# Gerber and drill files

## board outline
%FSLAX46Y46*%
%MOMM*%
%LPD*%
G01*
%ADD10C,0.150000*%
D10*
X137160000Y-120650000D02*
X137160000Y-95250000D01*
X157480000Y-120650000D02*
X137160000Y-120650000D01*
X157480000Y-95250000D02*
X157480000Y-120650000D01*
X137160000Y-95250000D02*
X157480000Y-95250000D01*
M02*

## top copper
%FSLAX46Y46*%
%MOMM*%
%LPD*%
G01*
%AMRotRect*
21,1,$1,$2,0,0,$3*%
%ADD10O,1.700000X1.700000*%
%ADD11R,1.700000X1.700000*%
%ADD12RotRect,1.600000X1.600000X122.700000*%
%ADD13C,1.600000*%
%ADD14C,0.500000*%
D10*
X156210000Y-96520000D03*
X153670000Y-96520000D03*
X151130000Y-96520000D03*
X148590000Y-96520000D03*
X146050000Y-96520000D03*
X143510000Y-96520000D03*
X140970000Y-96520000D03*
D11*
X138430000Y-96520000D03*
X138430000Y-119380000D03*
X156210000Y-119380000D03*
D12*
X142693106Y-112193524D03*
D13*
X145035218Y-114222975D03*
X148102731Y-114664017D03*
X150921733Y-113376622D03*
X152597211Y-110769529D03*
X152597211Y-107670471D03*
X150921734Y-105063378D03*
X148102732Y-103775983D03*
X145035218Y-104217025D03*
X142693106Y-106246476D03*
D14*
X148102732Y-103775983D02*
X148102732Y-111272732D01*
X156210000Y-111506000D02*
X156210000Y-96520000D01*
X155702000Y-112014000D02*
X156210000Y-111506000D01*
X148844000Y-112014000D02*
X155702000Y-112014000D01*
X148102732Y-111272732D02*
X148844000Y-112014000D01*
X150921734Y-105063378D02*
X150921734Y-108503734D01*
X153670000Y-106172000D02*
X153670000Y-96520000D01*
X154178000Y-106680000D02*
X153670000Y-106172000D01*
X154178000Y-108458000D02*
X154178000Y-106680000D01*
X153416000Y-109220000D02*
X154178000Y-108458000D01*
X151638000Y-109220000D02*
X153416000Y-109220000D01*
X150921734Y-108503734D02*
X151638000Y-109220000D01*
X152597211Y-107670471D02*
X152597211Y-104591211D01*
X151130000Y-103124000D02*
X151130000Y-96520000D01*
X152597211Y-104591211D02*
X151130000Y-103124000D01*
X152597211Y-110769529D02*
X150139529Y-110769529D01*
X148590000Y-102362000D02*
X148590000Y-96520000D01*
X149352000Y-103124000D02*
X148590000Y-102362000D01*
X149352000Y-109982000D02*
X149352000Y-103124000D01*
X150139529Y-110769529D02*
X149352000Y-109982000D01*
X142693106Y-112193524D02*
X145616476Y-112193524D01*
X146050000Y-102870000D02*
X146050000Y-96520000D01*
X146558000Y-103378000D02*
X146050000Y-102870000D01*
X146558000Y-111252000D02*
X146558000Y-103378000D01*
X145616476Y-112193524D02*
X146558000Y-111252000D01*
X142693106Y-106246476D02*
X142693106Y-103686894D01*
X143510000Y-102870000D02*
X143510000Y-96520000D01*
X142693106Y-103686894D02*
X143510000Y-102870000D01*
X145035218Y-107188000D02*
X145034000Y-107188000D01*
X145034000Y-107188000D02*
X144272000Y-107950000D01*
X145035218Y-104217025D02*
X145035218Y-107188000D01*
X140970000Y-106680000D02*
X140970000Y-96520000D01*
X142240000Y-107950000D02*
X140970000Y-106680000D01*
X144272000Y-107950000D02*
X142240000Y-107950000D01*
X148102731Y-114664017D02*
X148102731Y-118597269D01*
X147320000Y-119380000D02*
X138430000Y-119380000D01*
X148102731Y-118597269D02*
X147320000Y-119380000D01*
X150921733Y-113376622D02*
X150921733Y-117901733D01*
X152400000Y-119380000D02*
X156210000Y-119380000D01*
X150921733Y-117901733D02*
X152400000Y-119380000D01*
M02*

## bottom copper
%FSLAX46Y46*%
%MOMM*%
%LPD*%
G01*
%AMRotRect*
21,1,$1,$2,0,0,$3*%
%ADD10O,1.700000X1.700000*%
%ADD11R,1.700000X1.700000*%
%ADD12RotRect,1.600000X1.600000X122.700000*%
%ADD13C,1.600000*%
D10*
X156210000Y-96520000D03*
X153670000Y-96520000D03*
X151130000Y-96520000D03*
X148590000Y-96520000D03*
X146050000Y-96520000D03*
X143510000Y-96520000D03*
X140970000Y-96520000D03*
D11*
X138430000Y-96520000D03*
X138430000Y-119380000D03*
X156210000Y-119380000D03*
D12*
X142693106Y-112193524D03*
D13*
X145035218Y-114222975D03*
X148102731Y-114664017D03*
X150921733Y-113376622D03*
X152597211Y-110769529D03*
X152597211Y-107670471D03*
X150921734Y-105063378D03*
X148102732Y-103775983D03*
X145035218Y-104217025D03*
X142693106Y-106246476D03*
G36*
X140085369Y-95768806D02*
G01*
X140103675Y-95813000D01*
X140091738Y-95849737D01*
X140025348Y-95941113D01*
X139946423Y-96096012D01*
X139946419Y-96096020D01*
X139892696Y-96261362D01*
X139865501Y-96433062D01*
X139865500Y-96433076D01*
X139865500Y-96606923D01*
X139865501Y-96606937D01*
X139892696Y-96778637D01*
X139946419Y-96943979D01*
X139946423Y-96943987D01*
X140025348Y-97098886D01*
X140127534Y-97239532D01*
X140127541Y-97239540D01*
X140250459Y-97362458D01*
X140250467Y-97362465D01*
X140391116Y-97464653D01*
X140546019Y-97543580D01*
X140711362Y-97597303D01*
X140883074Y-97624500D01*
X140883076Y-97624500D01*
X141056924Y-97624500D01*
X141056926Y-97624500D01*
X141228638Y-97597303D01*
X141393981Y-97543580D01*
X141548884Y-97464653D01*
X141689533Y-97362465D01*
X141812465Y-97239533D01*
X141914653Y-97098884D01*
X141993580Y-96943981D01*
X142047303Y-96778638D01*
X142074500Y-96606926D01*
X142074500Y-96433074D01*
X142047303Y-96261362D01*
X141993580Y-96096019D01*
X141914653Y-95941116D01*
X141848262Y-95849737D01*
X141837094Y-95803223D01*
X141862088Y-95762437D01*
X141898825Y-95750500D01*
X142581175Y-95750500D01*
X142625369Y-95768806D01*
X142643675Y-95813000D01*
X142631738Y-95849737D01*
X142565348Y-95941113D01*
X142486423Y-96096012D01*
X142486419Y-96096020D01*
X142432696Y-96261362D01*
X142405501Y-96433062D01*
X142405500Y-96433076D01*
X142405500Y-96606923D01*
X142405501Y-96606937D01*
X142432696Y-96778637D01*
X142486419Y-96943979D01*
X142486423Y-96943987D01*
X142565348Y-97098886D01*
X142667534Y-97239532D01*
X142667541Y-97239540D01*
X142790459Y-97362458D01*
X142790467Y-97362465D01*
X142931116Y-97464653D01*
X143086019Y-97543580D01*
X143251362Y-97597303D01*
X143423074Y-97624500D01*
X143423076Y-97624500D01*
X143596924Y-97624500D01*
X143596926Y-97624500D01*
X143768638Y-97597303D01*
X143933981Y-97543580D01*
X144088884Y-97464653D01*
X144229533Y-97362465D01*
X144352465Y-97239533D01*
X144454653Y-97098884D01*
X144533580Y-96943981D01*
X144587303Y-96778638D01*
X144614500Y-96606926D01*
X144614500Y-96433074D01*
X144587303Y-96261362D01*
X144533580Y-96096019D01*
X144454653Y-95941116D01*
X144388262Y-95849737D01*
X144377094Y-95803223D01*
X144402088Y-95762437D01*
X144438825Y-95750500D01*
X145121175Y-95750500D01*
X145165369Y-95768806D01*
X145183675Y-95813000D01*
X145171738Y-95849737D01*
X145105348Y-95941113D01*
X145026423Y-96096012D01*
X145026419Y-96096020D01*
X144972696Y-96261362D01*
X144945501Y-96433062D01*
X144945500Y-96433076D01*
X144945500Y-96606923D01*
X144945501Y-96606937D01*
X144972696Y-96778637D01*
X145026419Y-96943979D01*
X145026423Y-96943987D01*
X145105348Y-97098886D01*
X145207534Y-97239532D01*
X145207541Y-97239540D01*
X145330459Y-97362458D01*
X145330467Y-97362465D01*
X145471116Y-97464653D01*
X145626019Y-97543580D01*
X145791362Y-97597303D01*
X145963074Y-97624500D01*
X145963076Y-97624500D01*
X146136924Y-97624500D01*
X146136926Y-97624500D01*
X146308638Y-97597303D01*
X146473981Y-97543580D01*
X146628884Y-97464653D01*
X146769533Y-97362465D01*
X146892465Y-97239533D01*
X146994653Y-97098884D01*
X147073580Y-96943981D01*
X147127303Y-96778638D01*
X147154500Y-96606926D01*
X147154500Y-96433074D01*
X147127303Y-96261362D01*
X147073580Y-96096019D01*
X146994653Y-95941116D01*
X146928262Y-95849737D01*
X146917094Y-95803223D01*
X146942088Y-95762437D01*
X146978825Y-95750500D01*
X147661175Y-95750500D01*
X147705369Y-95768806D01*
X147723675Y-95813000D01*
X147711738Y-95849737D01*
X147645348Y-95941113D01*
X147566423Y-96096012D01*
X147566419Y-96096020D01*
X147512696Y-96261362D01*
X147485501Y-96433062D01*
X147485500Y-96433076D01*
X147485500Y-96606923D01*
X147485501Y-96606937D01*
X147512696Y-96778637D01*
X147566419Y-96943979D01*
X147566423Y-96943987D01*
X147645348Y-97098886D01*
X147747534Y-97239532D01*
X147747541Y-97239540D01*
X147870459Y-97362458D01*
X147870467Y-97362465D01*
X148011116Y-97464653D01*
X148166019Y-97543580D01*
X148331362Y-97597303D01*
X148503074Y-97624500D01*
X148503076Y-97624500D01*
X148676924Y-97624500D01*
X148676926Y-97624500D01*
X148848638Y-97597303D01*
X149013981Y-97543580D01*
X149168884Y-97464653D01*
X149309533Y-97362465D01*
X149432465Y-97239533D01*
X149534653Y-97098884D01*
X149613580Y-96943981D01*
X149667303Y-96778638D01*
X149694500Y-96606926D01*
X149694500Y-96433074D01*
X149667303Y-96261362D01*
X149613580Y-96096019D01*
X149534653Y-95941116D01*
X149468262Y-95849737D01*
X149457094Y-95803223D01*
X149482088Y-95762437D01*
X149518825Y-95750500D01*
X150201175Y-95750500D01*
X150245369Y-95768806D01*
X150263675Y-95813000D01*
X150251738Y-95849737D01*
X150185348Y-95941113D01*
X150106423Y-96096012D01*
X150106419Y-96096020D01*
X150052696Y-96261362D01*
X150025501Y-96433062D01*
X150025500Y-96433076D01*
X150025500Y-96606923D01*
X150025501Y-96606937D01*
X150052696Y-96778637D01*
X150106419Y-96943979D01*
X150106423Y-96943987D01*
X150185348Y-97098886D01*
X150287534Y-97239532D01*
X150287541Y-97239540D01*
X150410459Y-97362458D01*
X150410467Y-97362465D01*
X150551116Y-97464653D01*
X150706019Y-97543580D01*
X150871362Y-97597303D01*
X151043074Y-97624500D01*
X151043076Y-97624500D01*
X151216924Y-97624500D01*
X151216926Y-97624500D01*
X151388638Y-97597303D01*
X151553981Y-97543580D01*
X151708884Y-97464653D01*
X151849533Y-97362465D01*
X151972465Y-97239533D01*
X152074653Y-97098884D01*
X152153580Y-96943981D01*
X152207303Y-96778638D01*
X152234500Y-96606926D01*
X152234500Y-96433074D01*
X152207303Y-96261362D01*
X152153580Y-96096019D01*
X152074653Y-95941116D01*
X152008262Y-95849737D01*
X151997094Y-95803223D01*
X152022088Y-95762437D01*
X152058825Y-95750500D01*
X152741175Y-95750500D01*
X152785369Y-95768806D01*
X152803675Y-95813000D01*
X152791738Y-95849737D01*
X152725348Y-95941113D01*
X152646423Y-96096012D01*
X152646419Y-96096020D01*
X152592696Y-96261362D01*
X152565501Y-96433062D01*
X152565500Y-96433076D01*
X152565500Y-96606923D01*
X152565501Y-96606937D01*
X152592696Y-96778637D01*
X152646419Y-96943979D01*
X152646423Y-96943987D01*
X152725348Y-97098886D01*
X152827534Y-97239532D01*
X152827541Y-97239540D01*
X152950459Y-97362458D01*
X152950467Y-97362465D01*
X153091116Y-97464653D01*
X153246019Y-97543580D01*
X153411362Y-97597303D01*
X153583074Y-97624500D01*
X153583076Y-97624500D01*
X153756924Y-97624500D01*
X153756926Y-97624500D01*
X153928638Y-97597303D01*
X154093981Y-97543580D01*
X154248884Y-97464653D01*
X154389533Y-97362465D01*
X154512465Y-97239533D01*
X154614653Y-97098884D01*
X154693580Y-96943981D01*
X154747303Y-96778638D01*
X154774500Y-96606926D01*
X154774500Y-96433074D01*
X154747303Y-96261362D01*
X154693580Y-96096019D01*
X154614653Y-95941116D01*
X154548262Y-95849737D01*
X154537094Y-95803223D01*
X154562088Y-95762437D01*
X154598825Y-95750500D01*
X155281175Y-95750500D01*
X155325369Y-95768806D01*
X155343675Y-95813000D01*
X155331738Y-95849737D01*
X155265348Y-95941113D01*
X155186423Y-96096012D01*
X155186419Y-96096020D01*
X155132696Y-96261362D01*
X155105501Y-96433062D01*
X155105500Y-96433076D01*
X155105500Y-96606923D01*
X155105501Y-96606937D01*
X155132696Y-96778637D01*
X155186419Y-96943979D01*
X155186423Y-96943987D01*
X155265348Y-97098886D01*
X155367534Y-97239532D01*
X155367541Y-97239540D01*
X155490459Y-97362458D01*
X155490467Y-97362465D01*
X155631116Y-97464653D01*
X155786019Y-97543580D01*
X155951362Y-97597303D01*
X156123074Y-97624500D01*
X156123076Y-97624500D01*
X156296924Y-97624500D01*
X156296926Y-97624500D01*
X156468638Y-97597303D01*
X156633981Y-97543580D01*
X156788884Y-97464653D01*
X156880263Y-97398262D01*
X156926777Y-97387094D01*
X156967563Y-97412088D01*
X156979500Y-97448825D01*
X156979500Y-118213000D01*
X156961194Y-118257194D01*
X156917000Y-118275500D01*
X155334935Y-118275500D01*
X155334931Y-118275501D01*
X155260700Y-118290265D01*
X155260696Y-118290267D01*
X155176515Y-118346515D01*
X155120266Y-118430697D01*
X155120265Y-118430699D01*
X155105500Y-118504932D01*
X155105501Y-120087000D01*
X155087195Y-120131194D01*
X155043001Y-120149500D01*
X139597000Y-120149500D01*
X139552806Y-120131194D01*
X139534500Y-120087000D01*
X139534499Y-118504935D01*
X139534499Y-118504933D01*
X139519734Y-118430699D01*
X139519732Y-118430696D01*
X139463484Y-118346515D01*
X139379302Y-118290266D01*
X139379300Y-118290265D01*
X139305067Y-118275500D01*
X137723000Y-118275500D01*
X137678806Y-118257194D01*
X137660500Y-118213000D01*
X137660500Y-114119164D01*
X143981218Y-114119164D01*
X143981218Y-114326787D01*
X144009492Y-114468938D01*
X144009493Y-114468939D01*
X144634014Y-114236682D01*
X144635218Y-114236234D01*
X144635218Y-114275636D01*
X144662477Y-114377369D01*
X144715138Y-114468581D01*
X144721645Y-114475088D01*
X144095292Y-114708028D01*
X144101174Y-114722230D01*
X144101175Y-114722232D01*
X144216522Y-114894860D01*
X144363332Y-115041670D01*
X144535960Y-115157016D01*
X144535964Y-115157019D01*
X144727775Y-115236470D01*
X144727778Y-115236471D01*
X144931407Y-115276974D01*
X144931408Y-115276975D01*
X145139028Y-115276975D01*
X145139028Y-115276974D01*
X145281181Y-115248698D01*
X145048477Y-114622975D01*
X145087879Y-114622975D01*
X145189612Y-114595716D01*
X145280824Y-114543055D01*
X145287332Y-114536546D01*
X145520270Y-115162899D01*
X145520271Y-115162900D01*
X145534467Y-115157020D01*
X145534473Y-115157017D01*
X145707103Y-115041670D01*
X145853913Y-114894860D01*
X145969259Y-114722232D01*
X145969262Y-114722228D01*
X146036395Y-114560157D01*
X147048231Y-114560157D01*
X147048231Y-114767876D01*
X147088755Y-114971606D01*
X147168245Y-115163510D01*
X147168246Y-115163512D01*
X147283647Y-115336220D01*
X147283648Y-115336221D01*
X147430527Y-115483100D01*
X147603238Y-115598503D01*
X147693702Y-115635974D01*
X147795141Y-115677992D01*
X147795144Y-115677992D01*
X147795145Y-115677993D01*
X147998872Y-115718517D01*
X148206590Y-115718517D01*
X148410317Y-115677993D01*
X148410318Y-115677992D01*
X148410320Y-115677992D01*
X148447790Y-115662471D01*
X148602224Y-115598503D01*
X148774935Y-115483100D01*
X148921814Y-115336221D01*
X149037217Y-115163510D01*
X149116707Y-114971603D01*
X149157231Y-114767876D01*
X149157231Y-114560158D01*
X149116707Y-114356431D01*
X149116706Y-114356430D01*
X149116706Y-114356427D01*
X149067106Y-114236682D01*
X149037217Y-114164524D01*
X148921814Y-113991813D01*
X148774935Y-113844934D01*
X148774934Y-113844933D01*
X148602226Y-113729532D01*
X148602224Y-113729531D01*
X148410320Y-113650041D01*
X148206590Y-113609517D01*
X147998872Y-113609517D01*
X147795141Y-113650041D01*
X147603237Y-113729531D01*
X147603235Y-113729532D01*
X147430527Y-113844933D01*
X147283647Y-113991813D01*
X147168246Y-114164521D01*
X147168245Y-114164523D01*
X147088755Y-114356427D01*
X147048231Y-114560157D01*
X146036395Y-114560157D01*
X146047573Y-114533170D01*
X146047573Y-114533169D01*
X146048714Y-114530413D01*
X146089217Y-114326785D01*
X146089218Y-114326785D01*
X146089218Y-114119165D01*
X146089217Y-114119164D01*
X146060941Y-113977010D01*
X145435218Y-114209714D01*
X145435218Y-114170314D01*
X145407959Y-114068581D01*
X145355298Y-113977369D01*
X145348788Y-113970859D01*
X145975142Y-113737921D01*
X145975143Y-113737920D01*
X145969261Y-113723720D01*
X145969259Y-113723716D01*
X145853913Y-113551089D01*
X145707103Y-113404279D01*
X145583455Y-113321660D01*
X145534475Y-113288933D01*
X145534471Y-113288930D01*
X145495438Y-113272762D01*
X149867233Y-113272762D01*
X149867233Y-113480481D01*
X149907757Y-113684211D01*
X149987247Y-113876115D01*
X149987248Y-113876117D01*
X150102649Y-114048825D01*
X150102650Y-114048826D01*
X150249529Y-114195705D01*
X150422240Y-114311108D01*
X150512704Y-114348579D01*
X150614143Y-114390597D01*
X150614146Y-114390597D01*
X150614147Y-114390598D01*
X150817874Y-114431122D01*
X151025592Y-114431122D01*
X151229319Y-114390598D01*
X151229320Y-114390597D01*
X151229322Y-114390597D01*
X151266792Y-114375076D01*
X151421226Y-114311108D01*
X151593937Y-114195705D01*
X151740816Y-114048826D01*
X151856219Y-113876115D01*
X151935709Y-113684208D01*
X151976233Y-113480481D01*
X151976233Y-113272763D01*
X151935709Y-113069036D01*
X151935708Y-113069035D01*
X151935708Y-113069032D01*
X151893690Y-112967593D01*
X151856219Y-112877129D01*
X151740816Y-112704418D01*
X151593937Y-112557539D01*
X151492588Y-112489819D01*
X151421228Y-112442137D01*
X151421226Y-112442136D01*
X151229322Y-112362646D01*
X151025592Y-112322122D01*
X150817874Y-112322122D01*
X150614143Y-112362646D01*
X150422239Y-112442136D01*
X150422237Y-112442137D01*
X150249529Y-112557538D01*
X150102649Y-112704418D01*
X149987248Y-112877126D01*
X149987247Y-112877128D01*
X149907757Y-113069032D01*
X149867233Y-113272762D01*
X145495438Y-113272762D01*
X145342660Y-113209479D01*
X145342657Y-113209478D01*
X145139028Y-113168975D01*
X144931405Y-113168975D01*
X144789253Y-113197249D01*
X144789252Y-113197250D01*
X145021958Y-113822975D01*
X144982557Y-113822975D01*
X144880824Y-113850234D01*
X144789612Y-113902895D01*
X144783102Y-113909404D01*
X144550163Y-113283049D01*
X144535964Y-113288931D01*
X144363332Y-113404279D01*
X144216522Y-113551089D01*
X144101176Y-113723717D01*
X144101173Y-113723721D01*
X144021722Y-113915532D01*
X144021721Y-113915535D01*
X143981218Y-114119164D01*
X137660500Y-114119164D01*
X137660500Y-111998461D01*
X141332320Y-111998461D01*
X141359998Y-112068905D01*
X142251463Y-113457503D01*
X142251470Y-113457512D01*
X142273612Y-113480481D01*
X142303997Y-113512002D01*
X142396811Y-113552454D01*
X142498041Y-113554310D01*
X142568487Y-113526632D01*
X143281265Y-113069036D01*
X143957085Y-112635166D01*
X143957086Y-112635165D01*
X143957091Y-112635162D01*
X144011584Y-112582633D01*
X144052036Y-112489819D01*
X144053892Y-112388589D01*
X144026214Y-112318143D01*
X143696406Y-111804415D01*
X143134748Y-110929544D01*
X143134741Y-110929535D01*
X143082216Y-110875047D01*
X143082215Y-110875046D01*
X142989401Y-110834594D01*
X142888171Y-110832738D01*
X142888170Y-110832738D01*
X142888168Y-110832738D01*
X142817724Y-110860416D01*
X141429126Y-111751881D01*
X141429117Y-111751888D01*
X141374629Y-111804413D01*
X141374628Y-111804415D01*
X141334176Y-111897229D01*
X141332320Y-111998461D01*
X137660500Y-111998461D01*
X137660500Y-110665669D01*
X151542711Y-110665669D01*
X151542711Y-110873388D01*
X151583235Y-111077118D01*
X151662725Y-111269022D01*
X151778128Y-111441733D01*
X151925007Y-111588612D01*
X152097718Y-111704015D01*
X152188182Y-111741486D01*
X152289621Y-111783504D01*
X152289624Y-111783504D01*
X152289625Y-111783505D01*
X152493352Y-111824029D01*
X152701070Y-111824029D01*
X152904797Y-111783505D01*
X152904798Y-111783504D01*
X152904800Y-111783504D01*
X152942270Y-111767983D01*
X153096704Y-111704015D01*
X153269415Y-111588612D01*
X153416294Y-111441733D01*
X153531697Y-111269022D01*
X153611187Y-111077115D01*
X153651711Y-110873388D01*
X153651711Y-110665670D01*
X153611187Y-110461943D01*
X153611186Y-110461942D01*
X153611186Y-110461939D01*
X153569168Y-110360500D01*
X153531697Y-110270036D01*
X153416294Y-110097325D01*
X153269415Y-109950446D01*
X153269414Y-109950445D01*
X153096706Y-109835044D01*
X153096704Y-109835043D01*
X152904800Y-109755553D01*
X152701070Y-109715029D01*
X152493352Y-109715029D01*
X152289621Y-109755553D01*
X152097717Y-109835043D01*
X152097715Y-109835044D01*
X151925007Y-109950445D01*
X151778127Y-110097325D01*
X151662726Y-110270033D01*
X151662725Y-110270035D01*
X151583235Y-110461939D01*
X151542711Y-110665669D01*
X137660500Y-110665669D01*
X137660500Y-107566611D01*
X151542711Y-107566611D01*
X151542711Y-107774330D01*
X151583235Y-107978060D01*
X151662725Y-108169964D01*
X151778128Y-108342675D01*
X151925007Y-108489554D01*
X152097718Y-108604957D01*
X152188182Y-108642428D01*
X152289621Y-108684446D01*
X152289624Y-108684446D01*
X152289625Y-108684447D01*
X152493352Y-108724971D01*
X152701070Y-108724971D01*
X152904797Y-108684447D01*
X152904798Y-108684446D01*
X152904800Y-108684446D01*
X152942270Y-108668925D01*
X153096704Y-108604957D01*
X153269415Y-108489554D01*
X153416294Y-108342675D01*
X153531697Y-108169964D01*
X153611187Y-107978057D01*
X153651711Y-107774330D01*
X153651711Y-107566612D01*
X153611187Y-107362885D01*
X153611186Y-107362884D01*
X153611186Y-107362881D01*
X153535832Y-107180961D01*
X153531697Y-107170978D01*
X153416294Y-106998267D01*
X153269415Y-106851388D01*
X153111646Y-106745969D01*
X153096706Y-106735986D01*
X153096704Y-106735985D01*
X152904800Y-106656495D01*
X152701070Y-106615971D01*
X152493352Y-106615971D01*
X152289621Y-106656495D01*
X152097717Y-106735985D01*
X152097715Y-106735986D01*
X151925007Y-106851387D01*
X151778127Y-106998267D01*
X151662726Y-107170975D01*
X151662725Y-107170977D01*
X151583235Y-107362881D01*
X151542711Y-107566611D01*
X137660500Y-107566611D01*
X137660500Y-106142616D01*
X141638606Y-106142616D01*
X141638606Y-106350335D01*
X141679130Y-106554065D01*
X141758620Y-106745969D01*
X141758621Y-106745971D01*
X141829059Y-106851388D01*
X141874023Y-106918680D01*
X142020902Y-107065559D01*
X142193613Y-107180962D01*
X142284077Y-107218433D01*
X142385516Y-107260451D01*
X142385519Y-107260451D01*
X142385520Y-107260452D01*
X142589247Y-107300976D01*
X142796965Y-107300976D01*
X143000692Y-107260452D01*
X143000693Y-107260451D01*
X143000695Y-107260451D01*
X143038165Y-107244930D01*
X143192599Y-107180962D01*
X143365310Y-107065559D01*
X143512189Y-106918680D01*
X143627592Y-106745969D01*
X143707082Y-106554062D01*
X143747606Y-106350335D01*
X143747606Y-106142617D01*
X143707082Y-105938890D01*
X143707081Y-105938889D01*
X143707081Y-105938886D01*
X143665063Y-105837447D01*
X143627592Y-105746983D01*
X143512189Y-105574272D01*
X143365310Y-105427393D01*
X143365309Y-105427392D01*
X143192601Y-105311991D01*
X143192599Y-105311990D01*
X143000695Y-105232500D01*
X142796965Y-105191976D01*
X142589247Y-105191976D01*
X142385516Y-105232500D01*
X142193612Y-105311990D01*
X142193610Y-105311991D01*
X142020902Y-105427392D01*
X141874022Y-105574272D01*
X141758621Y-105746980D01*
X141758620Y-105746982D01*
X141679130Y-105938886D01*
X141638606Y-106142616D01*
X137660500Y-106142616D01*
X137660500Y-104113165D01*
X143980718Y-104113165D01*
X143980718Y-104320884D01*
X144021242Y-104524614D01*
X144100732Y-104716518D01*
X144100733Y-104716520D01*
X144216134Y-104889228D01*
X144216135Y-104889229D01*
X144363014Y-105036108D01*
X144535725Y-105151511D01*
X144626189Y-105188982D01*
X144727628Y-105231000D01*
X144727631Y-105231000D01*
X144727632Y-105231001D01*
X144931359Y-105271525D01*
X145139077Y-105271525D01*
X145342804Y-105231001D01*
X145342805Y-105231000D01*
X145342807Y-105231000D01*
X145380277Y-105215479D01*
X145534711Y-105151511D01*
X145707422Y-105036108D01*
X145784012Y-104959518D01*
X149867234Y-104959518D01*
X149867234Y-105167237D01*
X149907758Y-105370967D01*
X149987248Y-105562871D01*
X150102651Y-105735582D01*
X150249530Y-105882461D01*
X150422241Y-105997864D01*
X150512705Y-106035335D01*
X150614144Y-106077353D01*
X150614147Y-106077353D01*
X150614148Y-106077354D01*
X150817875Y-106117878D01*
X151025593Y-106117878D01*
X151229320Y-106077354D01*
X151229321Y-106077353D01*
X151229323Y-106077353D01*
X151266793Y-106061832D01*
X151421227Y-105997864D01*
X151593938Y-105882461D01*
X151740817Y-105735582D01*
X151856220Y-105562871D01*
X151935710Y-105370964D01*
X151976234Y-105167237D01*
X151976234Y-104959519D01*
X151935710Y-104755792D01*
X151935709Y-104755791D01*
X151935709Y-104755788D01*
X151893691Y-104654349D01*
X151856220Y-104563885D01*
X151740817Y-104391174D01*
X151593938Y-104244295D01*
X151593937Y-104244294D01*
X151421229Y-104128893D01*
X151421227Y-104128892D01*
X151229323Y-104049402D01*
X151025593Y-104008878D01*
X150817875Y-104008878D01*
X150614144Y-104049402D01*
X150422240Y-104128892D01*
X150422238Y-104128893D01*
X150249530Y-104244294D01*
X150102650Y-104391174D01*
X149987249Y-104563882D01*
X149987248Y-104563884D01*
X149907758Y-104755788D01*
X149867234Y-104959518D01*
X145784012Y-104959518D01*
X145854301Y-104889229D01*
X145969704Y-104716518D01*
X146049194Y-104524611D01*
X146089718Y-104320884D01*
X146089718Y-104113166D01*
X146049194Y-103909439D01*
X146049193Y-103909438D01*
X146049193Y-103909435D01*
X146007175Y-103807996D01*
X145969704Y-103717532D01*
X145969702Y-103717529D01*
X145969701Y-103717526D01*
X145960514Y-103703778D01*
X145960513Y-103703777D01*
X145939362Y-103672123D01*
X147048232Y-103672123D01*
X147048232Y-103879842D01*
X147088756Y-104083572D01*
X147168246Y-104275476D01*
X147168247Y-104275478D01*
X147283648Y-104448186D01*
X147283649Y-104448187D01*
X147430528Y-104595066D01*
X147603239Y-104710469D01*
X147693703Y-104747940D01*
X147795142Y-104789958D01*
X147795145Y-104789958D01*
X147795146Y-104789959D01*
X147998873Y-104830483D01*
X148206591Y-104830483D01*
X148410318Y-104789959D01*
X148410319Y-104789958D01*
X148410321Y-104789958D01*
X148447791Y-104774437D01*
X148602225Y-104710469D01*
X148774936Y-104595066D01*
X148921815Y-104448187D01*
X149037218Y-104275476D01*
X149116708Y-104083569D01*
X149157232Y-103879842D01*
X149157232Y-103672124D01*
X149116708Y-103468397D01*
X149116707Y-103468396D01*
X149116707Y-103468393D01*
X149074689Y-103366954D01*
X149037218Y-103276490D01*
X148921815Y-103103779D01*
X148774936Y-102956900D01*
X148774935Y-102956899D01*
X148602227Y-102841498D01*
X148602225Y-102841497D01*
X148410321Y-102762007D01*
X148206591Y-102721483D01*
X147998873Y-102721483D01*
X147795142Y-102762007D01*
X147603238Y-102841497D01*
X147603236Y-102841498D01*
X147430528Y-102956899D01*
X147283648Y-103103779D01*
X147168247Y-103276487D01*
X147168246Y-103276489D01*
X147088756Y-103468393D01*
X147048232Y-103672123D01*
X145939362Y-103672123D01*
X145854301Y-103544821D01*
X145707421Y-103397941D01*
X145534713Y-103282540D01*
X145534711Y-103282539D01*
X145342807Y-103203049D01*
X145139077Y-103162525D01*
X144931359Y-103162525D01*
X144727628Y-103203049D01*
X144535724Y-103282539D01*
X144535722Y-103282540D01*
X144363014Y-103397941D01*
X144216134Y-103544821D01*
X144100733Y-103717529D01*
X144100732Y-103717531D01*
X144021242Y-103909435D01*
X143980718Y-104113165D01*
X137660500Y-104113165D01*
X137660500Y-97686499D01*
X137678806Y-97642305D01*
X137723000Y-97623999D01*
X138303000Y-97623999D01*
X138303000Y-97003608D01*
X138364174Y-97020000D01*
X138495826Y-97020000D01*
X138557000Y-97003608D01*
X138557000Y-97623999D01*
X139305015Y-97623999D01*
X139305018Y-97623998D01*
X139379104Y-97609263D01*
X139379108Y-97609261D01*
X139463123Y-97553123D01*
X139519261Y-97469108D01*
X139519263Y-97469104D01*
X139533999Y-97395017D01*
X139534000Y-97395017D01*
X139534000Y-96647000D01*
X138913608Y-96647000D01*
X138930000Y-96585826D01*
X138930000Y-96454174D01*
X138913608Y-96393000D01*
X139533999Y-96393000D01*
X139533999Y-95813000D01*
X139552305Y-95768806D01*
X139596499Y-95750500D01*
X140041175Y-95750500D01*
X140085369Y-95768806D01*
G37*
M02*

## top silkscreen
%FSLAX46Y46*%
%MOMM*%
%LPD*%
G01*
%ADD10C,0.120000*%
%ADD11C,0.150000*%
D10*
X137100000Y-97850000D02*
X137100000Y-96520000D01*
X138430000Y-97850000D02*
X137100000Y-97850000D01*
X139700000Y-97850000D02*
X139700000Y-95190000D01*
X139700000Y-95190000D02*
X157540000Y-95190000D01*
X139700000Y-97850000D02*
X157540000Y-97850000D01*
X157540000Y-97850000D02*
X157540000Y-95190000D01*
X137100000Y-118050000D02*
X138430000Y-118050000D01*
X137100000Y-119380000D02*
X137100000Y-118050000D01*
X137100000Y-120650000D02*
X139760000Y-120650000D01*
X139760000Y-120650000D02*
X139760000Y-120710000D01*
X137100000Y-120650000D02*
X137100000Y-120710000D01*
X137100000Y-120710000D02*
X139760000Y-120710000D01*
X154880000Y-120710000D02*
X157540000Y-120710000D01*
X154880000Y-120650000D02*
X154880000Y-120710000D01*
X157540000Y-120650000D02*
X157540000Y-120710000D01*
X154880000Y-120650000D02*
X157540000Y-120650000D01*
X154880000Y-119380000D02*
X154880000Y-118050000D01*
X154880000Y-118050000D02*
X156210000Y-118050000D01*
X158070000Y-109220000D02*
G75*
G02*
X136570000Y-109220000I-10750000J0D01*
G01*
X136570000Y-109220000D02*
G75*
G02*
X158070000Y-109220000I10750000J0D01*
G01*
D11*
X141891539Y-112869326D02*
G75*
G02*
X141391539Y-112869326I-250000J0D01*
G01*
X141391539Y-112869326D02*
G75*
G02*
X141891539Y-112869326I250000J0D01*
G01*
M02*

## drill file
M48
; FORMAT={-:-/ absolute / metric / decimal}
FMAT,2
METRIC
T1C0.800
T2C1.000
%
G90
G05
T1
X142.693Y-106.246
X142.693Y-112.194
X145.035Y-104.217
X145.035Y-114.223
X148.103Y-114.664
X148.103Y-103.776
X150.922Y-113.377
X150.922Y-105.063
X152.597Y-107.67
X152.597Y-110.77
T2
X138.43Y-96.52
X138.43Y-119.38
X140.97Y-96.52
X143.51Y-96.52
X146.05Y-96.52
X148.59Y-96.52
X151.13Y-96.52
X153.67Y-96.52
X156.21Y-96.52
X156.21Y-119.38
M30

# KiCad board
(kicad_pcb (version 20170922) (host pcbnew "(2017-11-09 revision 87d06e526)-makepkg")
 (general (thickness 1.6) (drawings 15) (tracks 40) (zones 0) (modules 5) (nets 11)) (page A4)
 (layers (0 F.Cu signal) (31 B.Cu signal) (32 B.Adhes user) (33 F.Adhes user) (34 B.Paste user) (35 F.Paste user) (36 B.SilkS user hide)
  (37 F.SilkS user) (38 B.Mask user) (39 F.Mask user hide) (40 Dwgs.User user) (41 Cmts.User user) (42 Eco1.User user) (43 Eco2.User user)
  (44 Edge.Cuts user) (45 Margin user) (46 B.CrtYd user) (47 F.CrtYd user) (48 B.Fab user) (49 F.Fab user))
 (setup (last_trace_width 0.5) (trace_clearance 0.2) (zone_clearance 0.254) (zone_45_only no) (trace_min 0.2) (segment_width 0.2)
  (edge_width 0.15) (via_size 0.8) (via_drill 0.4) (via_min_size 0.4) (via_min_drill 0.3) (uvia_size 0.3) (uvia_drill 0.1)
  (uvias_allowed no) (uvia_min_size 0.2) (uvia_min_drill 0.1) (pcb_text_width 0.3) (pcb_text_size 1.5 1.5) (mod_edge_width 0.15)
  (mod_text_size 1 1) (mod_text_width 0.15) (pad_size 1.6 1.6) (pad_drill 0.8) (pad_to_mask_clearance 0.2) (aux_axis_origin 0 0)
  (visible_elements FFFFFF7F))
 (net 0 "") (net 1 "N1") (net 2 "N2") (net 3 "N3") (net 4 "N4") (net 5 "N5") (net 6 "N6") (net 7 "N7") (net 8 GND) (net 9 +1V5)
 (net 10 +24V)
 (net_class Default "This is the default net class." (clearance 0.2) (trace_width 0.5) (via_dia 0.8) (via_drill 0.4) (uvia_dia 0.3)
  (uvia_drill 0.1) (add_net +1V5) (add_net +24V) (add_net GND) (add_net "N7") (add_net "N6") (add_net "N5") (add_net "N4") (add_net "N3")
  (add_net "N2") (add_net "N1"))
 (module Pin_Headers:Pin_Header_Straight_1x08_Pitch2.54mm (layer F.Cu) (at 138.43 96.52 90)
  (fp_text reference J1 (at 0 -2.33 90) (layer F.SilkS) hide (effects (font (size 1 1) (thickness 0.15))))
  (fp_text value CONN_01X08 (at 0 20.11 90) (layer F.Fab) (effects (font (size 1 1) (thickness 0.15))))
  (fp_line (start -1.33 -1.33) (end 0 -1.33) (layer F.SilkS) (width 0.12))
  (fp_line (start -1.33 0) (end -1.33 -1.33) (layer F.SilkS) (width 0.12))
  (fp_line (start -1.33 1.27) (end 1.33 1.27) (layer F.SilkS) (width 0.12))
  (fp_line (start 1.33 1.27) (end 1.33 19.11) (layer F.SilkS) (width 0.12))
  (fp_line (start -1.33 1.27) (end -1.33 19.11) (layer F.SilkS) (width 0.12))
  (fp_line (start -1.33 19.11) (end 1.33 19.11) (layer F.SilkS) (width 0.12))
  (pad 8 thru_hole oval (at 0 17.78 90) (size 1.7 1.7) (drill 1) (layers *.Cu *.Mask) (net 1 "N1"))
  (pad 7 thru_hole oval (at 0 15.24 90) (size 1.7 1.7) (drill 1) (layers *.Cu *.Mask) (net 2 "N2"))
  (pad 6 thru_hole oval (at 0 12.7 90) (size 1.7 1.7) (drill 1) (layers *.Cu *.Mask) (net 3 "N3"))
  (pad 5 thru_hole oval (at 0 10.16 90) (size 1.7 1.7) (drill 1) (layers *.Cu *.Mask) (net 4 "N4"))
  (pad 4 thru_hole oval (at 0 7.62 90) (size 1.7 1.7) (drill 1) (layers *.Cu *.Mask) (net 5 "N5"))
  (pad 3 thru_hole oval (at 0 5.08 90) (size 1.7 1.7) (drill 1) (layers *.Cu *.Mask) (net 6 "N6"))
  (pad 2 thru_hole oval (at 0 2.54 90) (size 1.7 1.7) (drill 1) (layers *.Cu *.Mask) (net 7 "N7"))
  (pad 1 thru_hole rect (at 0 0 90) (size 1.7 1.7) (drill 1) (layers *.Cu *.Mask) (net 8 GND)))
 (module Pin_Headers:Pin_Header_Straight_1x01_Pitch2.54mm (layer F.Cu) (at 138.43 119.38)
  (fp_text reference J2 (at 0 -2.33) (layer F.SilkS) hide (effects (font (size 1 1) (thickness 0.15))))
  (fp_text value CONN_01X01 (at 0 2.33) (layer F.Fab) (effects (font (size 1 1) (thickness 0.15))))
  (fp_line (start -1.33 -1.33) (end 0 -1.33) (layer F.SilkS) (width 0.12))
  (fp_line (start -1.33 0) (end -1.33 -1.33) (layer F.SilkS) (width 0.12))
  (fp_line (start -1.33 1.27) (end 1.33 1.27) (layer F.SilkS) (width 0.12))
  (fp_line (start 1.33 1.27) (end 1.33 1.33) (layer F.SilkS) (width 0.12))
  (fp_line (start -1.33 1.27) (end -1.33 1.33) (layer F.SilkS) (width 0.12))
  (fp_line (start -1.33 1.33) (end 1.33 1.33) (layer F.SilkS) (width 0.12))
  (pad 1 thru_hole rect (at 0 0) (size 1.7 1.7) (drill 1) (layers *.Cu *.Mask) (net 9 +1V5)))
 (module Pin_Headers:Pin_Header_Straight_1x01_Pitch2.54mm (layer F.Cu) (at 156.21 119.38)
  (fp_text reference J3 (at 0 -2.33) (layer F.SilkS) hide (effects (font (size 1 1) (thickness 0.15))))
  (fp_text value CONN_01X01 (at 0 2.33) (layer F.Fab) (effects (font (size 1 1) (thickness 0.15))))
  (fp_line (start -1.33 1.33) (end 1.33 1.33) (layer F.SilkS) (width 0.12))
  (fp_line (start -1.33 1.27) (end -1.33 1.33) (layer F.SilkS) (width 0.12))
  (fp_line (start 1.33 1.27) (end 1.33 1.33) (layer F.SilkS) (width 0.12))
  (fp_line (start -1.33 1.27) (end 1.33 1.27) (layer F.SilkS) (width 0.12))
  (fp_line (start -1.33 0) (end -1.33 -1.33) (layer F.SilkS) (width 0.12))
  (fp_line (start -1.33 -1.33) (end 0 -1.33) (layer F.SilkS) (width 0.12))
  (pad 1 thru_hole rect (at 0 0) (size 1.7 1.7) (drill 1) (layers *.Cu *.Mask) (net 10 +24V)))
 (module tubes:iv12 (layer F.Cu) (at 147.32 109.22 90)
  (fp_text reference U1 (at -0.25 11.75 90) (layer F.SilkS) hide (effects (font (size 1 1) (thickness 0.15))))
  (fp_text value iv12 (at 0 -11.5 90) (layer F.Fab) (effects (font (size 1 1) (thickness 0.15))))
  (fp_circle (center 0 0) (end 10.75 0) (layer F.SilkS) (width 0.12))
  (fp_circle (center -3.649326 -5.678461) (end -3.514165 -5.468148) (layer F.SilkS) (width 0.15))
  (pad 1 thru_hole rect (at -2.973524 -4.626894 122.7) (size 1.6 1.6) (drill 0.8) (layers *.Cu *.Mask) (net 5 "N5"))
  (pad 2 thru_hole circle (at -5.002975 -2.284782 155.4) (size 1.6 1.6) (drill 0.8) (layers *.Cu *.Mask) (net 8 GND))
  (pad 3 thru_hole circle (at -5.444017 0.782731 188.2) (size 1.6 1.6) (drill 0.8) (layers *.Cu *.Mask) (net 9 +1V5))
  (pad 4 thru_hole circle (at -4.156622 3.601733 220.9) (size 1.6 1.6) (drill 0.8) (layers *.Cu *.Mask) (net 10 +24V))
  (pad 5 thru_hole circle (at -1.549529 5.277211 253.6) (size 1.6 1.6) (drill 0.8) (layers *.Cu *.Mask) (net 4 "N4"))
  (pad 6 thru_hole circle (at 1.549529 5.277211 286.3) (size 1.6 1.6) (drill 0.8) (layers *.Cu *.Mask) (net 3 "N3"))
  (pad 7 thru_hole circle (at 4.156622 3.601734 319.1) (size 1.6 1.6) (drill 0.8) (layers *.Cu *.Mask) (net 2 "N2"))
  (pad 8 thru_hole circle (at 5.444017 0.782732 351.8) (size 1.6 1.6) (drill 0.8) (layers *.Cu *.Mask) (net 1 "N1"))
  (pad 9 thru_hole circle (at 5.002975 -2.284782 24.5) (size 1.6 1.6) (drill 0.8) (layers *.Cu *.Mask) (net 7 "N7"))
  (pad 10 thru_hole circle (at 2.973524 -4.626894 57.2) (size 1.6 1.6) (drill 0.8) (layers *.Cu *.Mask) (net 6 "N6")))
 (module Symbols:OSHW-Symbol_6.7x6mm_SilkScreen (layer B.Cu) (at 147.32 109.601)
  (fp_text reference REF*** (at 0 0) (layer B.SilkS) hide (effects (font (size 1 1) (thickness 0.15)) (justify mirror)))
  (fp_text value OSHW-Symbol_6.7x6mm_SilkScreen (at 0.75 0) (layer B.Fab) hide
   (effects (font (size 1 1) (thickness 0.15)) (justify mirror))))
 (gr_line (start 137.16 120.65) (end 137.16 95.25) (angle 90) (layer Edge.Cuts) (width 0.15))
 (gr_line (start 157.48 120.65) (end 137.16 120.65) (angle 90) (layer Edge.Cuts) (width 0.15))
 (gr_line (start 157.48 95.25) (end 157.48 120.65) (angle 90) (layer Edge.Cuts) (width 0.15))
 (gr_line (start 137.16 95.25) (end 157.48 95.25) (angle 90) (layer Edge.Cuts) (width 0.15))
 (segment (start 148.102732 103.775983) (end 148.102732 111.272732) (width 0.5) (layer F.Cu) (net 1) (status 400000))
 (segment (start 156.21 111.506) (end 156.21 96.52) (width 0.5) (layer F.Cu) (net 1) (status 800000))
 (segment (start 155.702 112.014) (end 156.21 111.506) (width 0.5) (layer F.Cu) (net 1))
 (segment (start 148.844 112.014) (end 155.702 112.014) (width 0.5) (layer F.Cu) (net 1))
 (segment (start 148.102732 111.272732) (end 148.844 112.014) (width 0.5) (layer F.Cu) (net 1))
 (segment (start 150.921734 105.063378) (end 150.921734 108.503734) (width 0.5) (layer F.Cu) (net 2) (status 400000))
 (segment (start 153.67 106.172) (end 153.67 96.52) (width 0.5) (layer F.Cu) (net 2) (status 800000))
 (segment (start 154.178 106.68) (end 153.67 106.172) (width 0.5) (layer F.Cu) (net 2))
 (segment (start 154.178 108.458) (end 154.178 106.68) (width 0.5) (layer F.Cu) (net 2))
 (segment (start 153.416 109.22) (end 154.178 108.458) (width 0.5) (layer F.Cu) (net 2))
 (segment (start 151.638 109.22) (end 153.416 109.22) (width 0.5) (layer F.Cu) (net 2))
 (segment (start 150.921734 108.503734) (end 151.638 109.22) (width 0.5) (layer F.Cu) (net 2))
 (segment (start 152.597211 107.670471) (end 152.597211 104.591211) (width 0.5) (layer F.Cu) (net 3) (status 400000))
 (segment (start 151.13 103.124) (end 151.13 96.52) (width 0.5) (layer F.Cu) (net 3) (status 800000))
 (segment (start 152.597211 104.591211) (end 151.13 103.124) (width 0.5) (layer F.Cu) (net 3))
 (segment (start 152.597211 110.769529) (end 150.139529 110.769529) (width 0.5) (layer F.Cu) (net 4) (status 400000))
 (segment (start 148.59 102.362) (end 148.59 96.52) (width 0.5) (layer F.Cu) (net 4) (status 800000))
 (segment (start 149.352 103.124) (end 148.59 102.362) (width 0.5) (layer F.Cu) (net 4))
 (segment (start 149.352 109.982) (end 149.352 103.124) (width 0.5) (layer F.Cu) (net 4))
 (segment (start 150.139529 110.769529) (end 149.352 109.982) (width 0.5) (layer F.Cu) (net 4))
 (segment (start 142.693106 112.193524) (end 145.616476 112.193524) (width 0.5) (layer F.Cu) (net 5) (status 400000))
 (segment (start 146.05 102.87) (end 146.05 96.52) (width 0.5) (layer F.Cu) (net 5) (status 800000))
 (segment (start 146.558 103.378) (end 146.05 102.87) (width 0.5) (layer F.Cu) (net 5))
 (segment (start 146.558 111.252) (end 146.558 103.378) (width 0.5) (layer F.Cu) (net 5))
 (segment (start 145.616476 112.193524) (end 146.558 111.252) (width 0.5) (layer F.Cu) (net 5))
 (segment (start 142.693106 106.246476) (end 142.693106 103.686894) (width 0.5) (layer F.Cu) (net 6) (status 400000))
 (segment (start 143.51 102.87) (end 143.51 96.52) (width 0.5) (layer F.Cu) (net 6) (status 800000))
 (segment (start 142.693106 103.686894) (end 143.51 102.87) (width 0.5) (layer F.Cu) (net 6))
 (segment (start 145.035218 107.188) (end 145.034 107.188) (width 0.5) (layer F.Cu) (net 7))
 (segment (start 145.034 107.188) (end 144.272 107.95) (width 0.5) (layer F.Cu) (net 7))
 (segment (start 145.035218 104.217025) (end 145.035218 107.188) (width 0.5) (layer F.Cu) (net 7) (status 400000))
 (segment (start 140.97 106.68) (end 140.97 96.52) (width 0.5) (layer F.Cu) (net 7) (status 800000))
 (segment (start 142.24 107.95) (end 140.97 106.68) (width 0.5) (layer F.Cu) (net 7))
 (segment (start 144.272 107.95) (end 142.24 107.95) (width 0.5) (layer F.Cu) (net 7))
 (segment (start 148.102731 114.664017) (end 148.102731 118.597269) (width 0.5) (layer F.Cu) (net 9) (status 400000))
 (segment (start 147.32 119.38) (end 138.43 119.38) (width 0.5) (layer F.Cu) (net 9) (status 800000))
 (segment (start 148.102731 118.597269) (end 147.32 119.38) (width 0.5) (layer F.Cu) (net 9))
 (segment (start 150.921733 113.376622) (end 150.921733 117.901733) (width 0.5) (layer F.Cu) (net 10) (status 400000))
 (segment (start 152.4 119.38) (end 156.21 119.38) (width 0.5) (layer F.Cu) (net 10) (status 800000))
 (segment (start 150.921733 117.901733) (end 152.4 119.38) (width 0.5) (layer F.Cu) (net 10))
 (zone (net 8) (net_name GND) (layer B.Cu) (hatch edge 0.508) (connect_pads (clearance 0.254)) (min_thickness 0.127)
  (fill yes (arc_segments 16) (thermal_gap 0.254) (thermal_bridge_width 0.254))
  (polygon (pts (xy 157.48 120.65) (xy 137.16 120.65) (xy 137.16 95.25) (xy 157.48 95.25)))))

